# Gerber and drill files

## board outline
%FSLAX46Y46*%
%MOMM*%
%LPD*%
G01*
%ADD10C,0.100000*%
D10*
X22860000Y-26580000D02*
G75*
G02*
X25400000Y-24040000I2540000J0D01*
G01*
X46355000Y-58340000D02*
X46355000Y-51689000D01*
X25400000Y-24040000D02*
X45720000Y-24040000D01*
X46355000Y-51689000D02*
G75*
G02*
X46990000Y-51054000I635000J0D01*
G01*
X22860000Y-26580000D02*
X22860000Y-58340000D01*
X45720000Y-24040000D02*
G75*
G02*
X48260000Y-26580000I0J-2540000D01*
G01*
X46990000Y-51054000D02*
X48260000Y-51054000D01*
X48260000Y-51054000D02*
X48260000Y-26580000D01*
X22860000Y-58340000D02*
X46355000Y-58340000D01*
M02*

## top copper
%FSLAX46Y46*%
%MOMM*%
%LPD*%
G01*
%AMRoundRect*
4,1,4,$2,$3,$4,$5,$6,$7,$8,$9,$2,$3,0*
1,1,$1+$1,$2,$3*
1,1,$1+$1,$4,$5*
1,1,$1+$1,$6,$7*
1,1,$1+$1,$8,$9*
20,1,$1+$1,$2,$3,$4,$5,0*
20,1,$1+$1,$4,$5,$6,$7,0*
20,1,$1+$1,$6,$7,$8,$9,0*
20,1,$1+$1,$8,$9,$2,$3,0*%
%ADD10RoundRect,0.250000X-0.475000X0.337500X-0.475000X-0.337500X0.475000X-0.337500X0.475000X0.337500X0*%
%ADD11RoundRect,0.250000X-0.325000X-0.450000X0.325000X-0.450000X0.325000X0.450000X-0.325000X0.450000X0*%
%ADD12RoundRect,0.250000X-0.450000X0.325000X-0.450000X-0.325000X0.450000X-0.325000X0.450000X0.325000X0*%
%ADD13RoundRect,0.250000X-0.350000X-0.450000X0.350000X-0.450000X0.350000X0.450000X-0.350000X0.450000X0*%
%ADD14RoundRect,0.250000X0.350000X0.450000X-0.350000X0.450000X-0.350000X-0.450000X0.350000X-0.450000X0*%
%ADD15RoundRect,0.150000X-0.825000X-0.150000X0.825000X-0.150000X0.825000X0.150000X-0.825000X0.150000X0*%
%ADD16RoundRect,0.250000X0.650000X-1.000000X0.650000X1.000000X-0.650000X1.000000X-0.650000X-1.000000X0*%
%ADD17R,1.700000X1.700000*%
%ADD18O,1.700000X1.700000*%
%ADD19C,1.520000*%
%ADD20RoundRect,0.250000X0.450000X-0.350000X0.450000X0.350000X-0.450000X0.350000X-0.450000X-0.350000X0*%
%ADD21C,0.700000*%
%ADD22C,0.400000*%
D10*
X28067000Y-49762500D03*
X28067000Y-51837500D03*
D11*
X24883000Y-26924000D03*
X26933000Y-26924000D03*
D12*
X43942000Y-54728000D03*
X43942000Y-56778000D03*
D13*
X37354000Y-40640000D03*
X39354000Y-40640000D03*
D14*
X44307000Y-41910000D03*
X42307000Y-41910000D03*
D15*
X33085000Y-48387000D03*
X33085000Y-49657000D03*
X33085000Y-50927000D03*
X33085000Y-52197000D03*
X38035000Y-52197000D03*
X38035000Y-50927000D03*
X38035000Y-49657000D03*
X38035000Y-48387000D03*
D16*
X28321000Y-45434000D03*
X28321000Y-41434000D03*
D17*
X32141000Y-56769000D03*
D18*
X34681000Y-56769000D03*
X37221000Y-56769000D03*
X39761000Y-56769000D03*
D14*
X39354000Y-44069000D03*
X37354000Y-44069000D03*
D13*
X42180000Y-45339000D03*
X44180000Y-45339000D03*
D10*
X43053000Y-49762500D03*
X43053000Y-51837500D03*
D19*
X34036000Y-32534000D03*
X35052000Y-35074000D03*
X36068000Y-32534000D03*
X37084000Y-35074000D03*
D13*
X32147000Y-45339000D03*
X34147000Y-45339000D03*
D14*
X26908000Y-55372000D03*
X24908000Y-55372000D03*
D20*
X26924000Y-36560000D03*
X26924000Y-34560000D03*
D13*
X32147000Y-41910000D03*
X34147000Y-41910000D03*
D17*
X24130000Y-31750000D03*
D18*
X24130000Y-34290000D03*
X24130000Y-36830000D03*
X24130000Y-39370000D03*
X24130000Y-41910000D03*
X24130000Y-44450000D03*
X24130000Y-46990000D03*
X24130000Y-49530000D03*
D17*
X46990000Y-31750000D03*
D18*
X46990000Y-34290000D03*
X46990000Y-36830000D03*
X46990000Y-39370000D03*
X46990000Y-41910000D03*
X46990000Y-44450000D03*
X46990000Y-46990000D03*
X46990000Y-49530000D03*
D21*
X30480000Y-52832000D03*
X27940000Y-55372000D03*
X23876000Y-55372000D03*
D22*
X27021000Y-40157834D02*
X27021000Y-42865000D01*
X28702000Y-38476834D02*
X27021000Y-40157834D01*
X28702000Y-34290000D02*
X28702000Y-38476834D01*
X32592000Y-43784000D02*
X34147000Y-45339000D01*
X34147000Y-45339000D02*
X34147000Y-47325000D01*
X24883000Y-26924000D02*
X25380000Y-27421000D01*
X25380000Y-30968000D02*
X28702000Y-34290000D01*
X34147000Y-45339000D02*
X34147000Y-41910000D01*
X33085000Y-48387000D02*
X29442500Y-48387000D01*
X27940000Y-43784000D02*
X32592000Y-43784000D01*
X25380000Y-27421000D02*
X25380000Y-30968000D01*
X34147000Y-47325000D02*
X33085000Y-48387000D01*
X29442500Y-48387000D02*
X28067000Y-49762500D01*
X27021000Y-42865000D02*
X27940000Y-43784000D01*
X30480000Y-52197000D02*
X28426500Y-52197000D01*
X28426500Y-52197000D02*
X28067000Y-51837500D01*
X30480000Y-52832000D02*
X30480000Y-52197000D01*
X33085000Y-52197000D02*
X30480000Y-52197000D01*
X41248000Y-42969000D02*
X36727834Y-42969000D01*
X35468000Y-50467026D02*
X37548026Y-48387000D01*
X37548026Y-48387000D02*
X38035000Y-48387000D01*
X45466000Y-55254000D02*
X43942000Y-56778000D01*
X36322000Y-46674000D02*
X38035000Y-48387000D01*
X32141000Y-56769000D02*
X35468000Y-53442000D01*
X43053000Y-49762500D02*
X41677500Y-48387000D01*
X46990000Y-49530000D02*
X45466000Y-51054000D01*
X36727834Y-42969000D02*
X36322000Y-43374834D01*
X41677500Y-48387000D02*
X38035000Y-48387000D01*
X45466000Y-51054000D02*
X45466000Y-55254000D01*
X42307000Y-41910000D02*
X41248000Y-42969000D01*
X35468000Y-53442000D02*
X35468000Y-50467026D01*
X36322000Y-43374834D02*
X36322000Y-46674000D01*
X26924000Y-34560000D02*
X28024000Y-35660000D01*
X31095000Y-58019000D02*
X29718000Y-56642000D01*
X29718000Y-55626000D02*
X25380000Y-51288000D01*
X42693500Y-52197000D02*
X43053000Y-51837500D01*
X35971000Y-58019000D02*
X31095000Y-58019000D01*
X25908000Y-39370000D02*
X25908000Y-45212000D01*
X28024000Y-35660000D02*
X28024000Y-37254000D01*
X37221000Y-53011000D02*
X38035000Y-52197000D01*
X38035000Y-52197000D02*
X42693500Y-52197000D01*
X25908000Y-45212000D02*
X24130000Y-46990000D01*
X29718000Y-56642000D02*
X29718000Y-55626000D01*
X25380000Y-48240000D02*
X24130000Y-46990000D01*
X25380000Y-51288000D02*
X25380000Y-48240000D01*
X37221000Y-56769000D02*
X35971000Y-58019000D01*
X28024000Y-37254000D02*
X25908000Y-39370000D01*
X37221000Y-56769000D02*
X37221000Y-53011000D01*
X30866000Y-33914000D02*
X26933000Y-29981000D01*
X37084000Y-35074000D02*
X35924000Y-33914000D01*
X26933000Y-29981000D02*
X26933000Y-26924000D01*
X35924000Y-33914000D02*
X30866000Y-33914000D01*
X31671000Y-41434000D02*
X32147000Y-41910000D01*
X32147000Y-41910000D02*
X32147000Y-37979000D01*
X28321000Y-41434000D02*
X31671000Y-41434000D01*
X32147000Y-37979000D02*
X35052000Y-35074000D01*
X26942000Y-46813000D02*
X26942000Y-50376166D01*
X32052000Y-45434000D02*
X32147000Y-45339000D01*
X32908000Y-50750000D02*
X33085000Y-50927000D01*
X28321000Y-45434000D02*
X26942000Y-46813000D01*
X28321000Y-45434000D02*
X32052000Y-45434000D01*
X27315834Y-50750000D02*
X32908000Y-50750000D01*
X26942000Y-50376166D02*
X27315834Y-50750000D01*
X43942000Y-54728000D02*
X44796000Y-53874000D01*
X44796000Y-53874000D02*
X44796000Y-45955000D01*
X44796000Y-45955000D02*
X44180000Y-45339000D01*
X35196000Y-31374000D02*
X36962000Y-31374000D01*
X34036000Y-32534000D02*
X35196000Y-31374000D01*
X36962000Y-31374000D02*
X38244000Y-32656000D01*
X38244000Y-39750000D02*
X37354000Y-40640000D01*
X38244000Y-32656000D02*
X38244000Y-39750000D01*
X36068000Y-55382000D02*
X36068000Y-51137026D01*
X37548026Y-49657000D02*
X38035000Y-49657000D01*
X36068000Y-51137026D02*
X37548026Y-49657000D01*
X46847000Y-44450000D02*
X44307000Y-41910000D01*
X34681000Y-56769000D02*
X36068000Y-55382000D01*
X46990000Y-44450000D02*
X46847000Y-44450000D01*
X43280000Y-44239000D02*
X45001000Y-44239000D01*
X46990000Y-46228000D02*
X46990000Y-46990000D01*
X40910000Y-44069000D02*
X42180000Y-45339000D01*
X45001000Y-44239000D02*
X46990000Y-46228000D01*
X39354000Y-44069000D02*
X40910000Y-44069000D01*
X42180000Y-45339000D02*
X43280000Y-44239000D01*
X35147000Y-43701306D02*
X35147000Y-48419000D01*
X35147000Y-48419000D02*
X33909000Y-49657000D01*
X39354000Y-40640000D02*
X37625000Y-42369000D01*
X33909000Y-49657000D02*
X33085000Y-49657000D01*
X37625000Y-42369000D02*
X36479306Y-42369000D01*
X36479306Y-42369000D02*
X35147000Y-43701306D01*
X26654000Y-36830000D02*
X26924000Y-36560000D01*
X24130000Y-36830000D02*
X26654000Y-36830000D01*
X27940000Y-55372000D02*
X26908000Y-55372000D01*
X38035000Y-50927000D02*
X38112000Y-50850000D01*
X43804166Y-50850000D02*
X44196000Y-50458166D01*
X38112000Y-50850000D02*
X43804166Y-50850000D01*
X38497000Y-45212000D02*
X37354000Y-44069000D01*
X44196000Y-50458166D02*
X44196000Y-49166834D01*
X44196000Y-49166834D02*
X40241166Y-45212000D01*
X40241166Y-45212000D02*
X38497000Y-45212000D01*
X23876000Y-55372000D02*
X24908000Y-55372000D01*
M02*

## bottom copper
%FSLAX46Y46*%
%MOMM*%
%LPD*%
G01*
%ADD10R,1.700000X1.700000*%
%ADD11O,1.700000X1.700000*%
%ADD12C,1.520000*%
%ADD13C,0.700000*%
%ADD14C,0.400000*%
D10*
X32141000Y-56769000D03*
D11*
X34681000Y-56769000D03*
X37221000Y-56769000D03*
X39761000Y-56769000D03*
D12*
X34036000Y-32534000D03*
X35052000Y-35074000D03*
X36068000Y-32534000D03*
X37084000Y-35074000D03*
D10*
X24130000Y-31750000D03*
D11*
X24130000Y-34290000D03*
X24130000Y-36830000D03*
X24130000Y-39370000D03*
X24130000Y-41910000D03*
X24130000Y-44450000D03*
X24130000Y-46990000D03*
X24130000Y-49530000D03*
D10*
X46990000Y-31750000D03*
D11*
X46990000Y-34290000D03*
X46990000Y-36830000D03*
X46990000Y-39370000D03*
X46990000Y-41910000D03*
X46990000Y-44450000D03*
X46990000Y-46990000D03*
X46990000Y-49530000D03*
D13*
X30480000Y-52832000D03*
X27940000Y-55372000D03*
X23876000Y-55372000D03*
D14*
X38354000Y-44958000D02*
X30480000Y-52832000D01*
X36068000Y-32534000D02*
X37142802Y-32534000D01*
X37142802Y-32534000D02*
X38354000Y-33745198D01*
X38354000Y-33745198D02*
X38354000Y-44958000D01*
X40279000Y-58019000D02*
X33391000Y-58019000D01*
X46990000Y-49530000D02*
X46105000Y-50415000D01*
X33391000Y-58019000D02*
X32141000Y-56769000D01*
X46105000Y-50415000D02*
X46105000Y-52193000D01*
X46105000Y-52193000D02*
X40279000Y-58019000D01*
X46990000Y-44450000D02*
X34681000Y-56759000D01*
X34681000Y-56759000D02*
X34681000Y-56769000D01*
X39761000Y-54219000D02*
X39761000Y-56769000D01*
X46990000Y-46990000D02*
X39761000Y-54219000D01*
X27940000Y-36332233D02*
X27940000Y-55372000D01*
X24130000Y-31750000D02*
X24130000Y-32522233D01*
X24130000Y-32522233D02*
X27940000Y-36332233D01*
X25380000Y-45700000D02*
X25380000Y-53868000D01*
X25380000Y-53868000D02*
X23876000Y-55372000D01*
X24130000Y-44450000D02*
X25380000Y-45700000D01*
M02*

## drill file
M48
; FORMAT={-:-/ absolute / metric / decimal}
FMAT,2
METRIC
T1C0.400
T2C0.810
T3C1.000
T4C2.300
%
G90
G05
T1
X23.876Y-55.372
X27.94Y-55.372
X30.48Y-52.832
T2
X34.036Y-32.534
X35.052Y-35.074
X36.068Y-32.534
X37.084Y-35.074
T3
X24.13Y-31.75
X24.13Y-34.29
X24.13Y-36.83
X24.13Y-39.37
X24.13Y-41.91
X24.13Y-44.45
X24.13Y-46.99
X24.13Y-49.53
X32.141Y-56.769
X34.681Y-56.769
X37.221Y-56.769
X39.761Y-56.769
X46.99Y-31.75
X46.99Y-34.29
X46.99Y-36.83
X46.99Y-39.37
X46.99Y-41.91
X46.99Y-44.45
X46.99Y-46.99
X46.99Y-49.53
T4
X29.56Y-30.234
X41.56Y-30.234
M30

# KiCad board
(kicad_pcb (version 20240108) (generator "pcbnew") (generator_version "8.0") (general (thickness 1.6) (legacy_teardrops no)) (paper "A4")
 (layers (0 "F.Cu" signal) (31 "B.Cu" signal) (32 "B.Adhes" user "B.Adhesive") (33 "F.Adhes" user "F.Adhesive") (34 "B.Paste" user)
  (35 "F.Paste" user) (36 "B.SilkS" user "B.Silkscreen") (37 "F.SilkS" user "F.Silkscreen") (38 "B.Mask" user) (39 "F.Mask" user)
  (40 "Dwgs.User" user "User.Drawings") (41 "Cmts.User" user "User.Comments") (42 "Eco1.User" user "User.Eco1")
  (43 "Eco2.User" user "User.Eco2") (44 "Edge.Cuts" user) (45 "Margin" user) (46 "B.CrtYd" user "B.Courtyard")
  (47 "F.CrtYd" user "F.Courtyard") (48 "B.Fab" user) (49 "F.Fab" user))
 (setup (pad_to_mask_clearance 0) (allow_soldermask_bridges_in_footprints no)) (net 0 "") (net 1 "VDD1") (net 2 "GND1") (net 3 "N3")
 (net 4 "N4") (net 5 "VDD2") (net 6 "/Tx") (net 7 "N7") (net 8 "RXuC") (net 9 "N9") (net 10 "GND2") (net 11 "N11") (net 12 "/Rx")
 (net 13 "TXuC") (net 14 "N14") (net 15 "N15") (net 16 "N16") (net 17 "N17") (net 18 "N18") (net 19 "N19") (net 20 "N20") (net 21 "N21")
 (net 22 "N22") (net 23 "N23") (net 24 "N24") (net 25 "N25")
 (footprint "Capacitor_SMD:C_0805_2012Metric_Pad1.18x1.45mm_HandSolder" (layer "F.Cu") (at 28.067 50.8 -90)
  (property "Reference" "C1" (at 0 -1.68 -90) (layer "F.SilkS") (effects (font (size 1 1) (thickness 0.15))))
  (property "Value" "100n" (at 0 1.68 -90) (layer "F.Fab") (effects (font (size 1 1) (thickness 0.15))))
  (pad "1" smd roundrect (at -1.0375 0 270) (size 1.175 1.45) (layers "F.Cu" "F.Paste" "F.Mask") (roundrect_rratio 0.212766) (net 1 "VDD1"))
  (pad "2" smd roundrect (at 1.0375 0 270) (size 1.175 1.45) (layers "F.Cu" "F.Paste" "F.Mask") (roundrect_rratio 0.212766) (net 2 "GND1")))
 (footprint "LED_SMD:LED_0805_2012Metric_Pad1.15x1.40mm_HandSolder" (layer "F.Cu") (at 25.908 26.924)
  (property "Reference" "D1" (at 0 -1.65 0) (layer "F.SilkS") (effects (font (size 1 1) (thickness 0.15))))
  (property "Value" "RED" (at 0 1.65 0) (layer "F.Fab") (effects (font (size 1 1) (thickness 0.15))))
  (pad "1" smd roundrect (at -1.025 0) (size 1.15 1.4) (layers "F.Cu" "F.Paste" "F.Mask") (roundrect_rratio 0.217391) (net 1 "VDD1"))
  (pad "2" smd roundrect (at 1.025 0) (size 1.15 1.4) (layers "F.Cu" "F.Paste" "F.Mask") (roundrect_rratio 0.217391) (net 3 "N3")))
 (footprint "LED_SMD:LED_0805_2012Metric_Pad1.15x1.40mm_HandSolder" (layer "F.Cu") (at 43.942 55.753 -90)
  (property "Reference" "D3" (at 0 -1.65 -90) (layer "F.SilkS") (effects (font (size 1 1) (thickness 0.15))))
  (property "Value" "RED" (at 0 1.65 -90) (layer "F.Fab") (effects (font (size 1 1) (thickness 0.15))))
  (pad "1" smd roundrect (at -1.025 0 270) (size 1.15 1.4) (layers "F.Cu" "F.Paste" "F.Mask") (roundrect_rratio 0.217391) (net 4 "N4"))
  (pad "2" smd roundrect (at 1.025 0 270) (size 1.15 1.4) (layers "F.Cu" "F.Paste" "F.Mask") (roundrect_rratio 0.217391) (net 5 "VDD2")))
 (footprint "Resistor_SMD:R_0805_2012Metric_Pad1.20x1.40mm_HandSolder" (layer "F.Cu") (at 38.354 40.64)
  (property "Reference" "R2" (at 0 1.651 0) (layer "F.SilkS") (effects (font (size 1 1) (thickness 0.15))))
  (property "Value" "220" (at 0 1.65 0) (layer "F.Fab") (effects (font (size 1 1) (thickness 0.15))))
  (pad "1" smd roundrect (at -1 0) (size 1.2 1.4) (layers "F.Cu" "F.Paste" "F.Mask") (roundrect_rratio 0.208333) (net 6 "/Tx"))
  (pad "2" smd roundrect (at 1 0) (size 1.2 1.4) (layers "F.Cu" "F.Paste" "F.Mask") (roundrect_rratio 0.208333) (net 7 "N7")))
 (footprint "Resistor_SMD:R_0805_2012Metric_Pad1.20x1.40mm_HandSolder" (layer "F.Cu") (at 43.307 41.91 180)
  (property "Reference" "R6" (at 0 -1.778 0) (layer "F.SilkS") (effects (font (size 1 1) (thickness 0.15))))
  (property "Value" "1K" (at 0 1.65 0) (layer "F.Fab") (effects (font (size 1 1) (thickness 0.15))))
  (pad "1" smd roundrect (at -1 0 180) (size 1.2 1.4) (layers "F.Cu" "F.Paste" "F.Mask") (roundrect_rratio 0.208333) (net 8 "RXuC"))
  (pad "2" smd roundrect (at 1 0 180) (size 1.2 1.4) (layers "F.Cu" "F.Paste" "F.Mask") (roundrect_rratio 0.208333) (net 5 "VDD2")))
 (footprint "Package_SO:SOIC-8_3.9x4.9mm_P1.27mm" (layer "F.Cu") (at 35.56 50.292)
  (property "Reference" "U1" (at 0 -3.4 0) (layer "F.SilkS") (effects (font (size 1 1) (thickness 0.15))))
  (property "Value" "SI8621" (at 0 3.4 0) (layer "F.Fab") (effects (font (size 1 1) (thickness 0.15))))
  (pad "1" smd roundrect (at -2.475 -1.905) (size 1.95 0.6) (layers "F.Cu" "F.Paste" "F.Mask") (roundrect_rratio 0.25) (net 1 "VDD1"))
  (pad "2" smd roundrect (at -2.475 -0.635) (size 1.95 0.6) (layers "F.Cu" "F.Paste" "F.Mask") (roundrect_rratio 0.25) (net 7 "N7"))
  (pad "3" smd roundrect (at -2.475 0.635) (size 1.95 0.6) (layers "F.Cu" "F.Paste" "F.Mask") (roundrect_rratio 0.25) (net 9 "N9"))
  (pad "4" smd roundrect (at -2.475 1.905) (size 1.95 0.6) (layers "F.Cu" "F.Paste" "F.Mask") (roundrect_rratio 0.25) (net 2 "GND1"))
  (pad "5" smd roundrect (at 2.475 1.905) (size 1.95 0.6) (layers "F.Cu" "F.Paste" "F.Mask") (roundrect_rratio 0.25) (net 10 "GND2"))
  (pad "6" smd roundrect (at 2.475 0.635) (size 1.95 0.6) (layers "F.Cu" "F.Paste" "F.Mask") (roundrect_rratio 0.25) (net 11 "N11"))
  (pad "7" smd roundrect (at 2.475 -0.635) (size 1.95 0.6) (layers "F.Cu" "F.Paste" "F.Mask") (roundrect_rratio 0.25) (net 8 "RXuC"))
  (pad "8" smd roundrect (at 2.475 -1.905) (size 1.95 0.6) (layers "F.Cu" "F.Paste" "F.Mask") (roundrect_rratio 0.25) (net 5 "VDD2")))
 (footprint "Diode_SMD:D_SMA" (layer "F.Cu") (at 28.321 43.434 90)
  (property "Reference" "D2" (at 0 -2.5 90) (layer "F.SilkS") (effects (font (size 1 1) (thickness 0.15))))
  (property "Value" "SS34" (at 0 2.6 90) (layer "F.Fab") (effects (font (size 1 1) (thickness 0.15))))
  (pad "1" smd roundrect (at -2 0 90) (size 2.5 1.8) (layers "F.Cu" "F.Paste" "F.Mask") (roundrect_rratio 0.1388888889) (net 9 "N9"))
  (pad "2" smd roundrect (at 2 0 90) (size 2.5 1.8) (layers "F.Cu" "F.Paste" "F.Mask") (roundrect_rratio 0.1388888889) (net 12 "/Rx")))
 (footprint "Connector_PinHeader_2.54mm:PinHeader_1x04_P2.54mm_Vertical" (layer "F.Cu") (at 32.141 56.769 90)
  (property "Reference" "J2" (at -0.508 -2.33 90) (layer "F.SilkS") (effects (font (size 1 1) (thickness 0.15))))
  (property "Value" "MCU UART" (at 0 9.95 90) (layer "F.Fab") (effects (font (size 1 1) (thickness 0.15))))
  (pad "1" thru_hole rect (at 0 0 90) (size 1.7 1.7) (drill 1) (layers "*.Cu" "*.Mask") (remove_unused_layers no) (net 5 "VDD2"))
  (pad "2" thru_hole oval (at 0 2.54 90) (size 1.7 1.7) (drill 1) (layers "*.Cu" "*.Mask") (remove_unused_layers no) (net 8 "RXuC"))
  (pad "3" thru_hole oval (at 0 5.08 90) (size 1.7 1.7) (drill 1) (layers "*.Cu" "*.Mask") (remove_unused_layers no) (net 10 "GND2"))
  (pad "4" thru_hole oval (at 0 7.62 90) (size 1.7 1.7) (drill 1) (layers "*.Cu" "*.Mask") (remove_unused_layers no) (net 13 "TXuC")))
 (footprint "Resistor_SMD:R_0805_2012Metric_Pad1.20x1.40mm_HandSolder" (layer "F.Cu") (at 38.354 44.069 180)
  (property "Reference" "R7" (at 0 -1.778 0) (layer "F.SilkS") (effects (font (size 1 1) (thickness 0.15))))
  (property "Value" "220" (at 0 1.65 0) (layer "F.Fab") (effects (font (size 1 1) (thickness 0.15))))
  (pad "1" smd roundrect (at -1 0 180) (size 1.2 1.4) (layers "F.Cu" "F.Paste" "F.Mask") (roundrect_rratio 0.208333) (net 13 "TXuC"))
  (pad "2" smd roundrect (at 1 0 180) (size 1.2 1.4) (layers "F.Cu" "F.Paste" "F.Mask") (roundrect_rratio 0.208333) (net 11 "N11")))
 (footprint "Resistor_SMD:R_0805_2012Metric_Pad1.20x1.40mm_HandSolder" (layer "F.Cu") (at 43.18 45.339)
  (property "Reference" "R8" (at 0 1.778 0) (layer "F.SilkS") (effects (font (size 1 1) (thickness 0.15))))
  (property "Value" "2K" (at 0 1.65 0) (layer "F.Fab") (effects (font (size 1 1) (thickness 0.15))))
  (pad "1" smd roundrect (at -1 0) (size 1.2 1.4) (layers "F.Cu" "F.Paste" "F.Mask") (roundrect_rratio 0.208333) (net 13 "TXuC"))
  (pad "2" smd roundrect (at 1 0) (size 1.2 1.4) (layers "F.Cu" "F.Paste" "F.Mask") (roundrect_rratio 0.208333) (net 4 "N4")))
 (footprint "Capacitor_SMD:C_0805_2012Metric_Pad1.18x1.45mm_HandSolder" (layer "F.Cu") (at 43.053 50.8 -90)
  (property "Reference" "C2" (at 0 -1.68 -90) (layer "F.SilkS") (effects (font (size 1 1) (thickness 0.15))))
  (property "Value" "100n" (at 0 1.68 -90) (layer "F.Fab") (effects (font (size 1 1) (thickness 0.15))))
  (pad "1" smd roundrect (at -1.0375 0 270) (size 1.175 1.45) (layers "F.Cu" "F.Paste" "F.Mask") (roundrect_rratio 0.212766) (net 5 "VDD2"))
  (pad "2" smd roundrect (at 1.0375 0 270) (size 1.175 1.45) (layers "F.Cu" "F.Paste" "F.Mask") (roundrect_rratio 0.212766) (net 10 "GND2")))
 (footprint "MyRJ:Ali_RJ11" (layer "F.Cu") (at 34.036 32.534 180)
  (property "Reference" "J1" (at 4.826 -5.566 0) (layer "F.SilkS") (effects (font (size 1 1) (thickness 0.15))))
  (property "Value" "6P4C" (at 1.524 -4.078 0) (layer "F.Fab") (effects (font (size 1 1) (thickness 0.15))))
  (pad "" np_thru_hole circle (at -7.524 2.3 180) (size 2.3 2.3) (drill 2.3) (layers "F&B.Cu" "*.Mask"))
  (pad "" np_thru_hole circle (at 4.476 2.3 180) (size 2.3 2.3) (drill 2.3) (layers "F&B.Cu" "*.Mask"))
  (pad "1" thru_hole circle (at 0 0) (size 1.52 1.52) (drill 0.81) (layers "*.Cu" "*.Mask") (remove_unused_layers no) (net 6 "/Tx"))
  (pad "2" thru_hole circle (at -1.016 -2.54) (size 1.52 1.52) (drill 0.81) (layers "*.Cu" "*.Mask") (remove_unused_layers no)
   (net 12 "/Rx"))
  (pad "3" thru_hole circle (at -2.032 0) (size 1.52 1.52) (drill 0.81) (layers "*.Cu" "*.Mask") (remove_unused_layers no) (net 2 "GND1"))
  (pad "4" thru_hole circle (at -3.048 -2.54) (size 1.52 1.52) (drill 0.81) (layers "*.Cu" "*.Mask") (remove_unused_layers no) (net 3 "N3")))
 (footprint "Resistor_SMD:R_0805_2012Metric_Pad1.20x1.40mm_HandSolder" (layer "F.Cu") (at 33.147 45.339)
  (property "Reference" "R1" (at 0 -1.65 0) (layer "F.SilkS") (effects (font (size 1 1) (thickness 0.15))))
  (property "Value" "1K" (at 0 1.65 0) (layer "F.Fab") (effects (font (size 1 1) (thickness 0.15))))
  (pad "1" smd roundrect (at -1 0) (size 1.2 1.4) (layers "F.Cu" "F.Paste" "F.Mask") (roundrect_rratio 0.208333) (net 9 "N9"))
  (pad "2" smd roundrect (at 1 0) (size 1.2 1.4) (layers "F.Cu" "F.Paste" "F.Mask") (roundrect_rratio 0.208333) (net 1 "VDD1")))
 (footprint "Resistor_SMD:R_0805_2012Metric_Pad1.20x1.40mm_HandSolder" (layer "F.Cu") (at 25.908 55.372 180)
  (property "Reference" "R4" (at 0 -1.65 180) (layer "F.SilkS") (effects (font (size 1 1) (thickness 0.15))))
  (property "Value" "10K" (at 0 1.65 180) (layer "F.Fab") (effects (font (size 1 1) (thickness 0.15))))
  (pad "1" smd roundrect (at -1 0 180) (size 1.2 1.4) (layers "F.Cu" "F.Paste" "F.Mask") (roundrect_rratio 0.208333) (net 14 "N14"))
  (pad "2" smd roundrect (at 1 0 180) (size 1.2 1.4) (layers "F.Cu" "F.Paste" "F.Mask") (roundrect_rratio 0.208333) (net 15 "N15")))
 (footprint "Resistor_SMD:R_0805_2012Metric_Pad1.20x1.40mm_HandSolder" (layer "F.Cu") (at 26.924 35.56 90)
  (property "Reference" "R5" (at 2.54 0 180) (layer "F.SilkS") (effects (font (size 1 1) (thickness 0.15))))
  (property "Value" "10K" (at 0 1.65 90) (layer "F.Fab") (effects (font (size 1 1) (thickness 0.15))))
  (pad "1" smd roundrect (at -1 0 90) (size 1.2 1.4) (layers "F.Cu" "F.Paste" "F.Mask") (roundrect_rratio 0.208333) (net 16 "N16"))
  (pad "2" smd roundrect (at 1 0 90) (size 1.2 1.4) (layers "F.Cu" "F.Paste" "F.Mask") (roundrect_rratio 0.208333) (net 10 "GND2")))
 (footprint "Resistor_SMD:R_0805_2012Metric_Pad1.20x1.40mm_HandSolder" (layer "F.Cu") (at 33.147 41.91)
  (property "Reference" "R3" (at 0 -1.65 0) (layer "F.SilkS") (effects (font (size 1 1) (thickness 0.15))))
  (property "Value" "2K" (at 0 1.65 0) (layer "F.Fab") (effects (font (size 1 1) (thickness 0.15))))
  (pad "1" smd roundrect (at -1 0) (size 1.2 1.4) (layers "F.Cu" "F.Paste" "F.Mask") (roundrect_rratio 0.208333) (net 12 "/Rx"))
  (pad "2" smd roundrect (at 1 0) (size 1.2 1.4) (layers "F.Cu" "F.Paste" "F.Mask") (roundrect_rratio 0.208333) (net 1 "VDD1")))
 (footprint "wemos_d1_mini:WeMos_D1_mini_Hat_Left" (layer "B.Cu") (at 24.13 31.75 180)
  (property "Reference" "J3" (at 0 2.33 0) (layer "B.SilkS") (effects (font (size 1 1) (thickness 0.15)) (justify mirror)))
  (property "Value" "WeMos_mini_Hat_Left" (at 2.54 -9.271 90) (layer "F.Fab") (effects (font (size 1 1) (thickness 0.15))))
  (pad "1" thru_hole rect (at 0 0 180) (size 1.7 1.7) (drill 1) (layers "*.Cu" "*.Mask") (remove_unused_layers no) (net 14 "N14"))
  (pad "2" thru_hole oval (at 0 -2.54 180) (size 1.7 1.7) (drill 1) (layers "*.Cu" "*.Mask") (remove_unused_layers no) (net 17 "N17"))
  (pad "3" thru_hole oval (at 0 -5.08 180) (size 1.7 1.7) (drill 1) (layers "*.Cu" "*.Mask") (remove_unused_layers no) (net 16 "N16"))
  (pad "4" thru_hole oval (at 0 -7.62 180) (size 1.7 1.7) (drill 1) (layers "*.Cu" "*.Mask") (remove_unused_layers no) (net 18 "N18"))
  (pad "5" thru_hole oval (at 0 -10.16 180) (size 1.7 1.7) (drill 1) (layers "*.Cu" "*.Mask") (remove_unused_layers no) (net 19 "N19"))
  (pad "6" thru_hole oval (at 0 -12.7 180) (size 1.7 1.7) (drill 1) (layers "*.Cu" "*.Mask") (remove_unused_layers no) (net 15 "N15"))
  (pad "7" thru_hole oval (at 0 -15.24 180) (size 1.7 1.7) (drill 1) (layers "*.Cu" "*.Mask") (remove_unused_layers no) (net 10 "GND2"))
  (pad "8" thru_hole oval (at 0 -17.78 180) (size 1.7 1.7) (drill 1) (layers "*.Cu" "*.Mask") (remove_unused_layers no) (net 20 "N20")))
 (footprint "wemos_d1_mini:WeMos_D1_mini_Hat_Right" (layer "B.Cu") (at 46.99 31.75 180)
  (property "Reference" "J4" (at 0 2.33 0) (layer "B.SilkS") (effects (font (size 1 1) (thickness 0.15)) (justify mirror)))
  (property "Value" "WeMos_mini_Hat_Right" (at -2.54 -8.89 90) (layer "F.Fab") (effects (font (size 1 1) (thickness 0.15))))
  (pad "1" thru_hole rect (at 0 0 180) (size 1.7 1.7) (drill 1) (layers "*.Cu" "*.Mask") (remove_unused_layers no) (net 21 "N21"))
  (pad "2" thru_hole oval (at 0 -2.54 180) (size 1.7 1.7) (drill 1) (layers "*.Cu" "*.Mask") (remove_unused_layers no) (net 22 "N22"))
  (pad "3" thru_hole oval (at 0 -5.08 180) (size 1.7 1.7) (drill 1) (layers "*.Cu" "*.Mask") (remove_unused_layers no) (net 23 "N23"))
  (pad "4" thru_hole oval (at 0 -7.62 180) (size 1.7 1.7) (drill 1) (layers "*.Cu" "*.Mask") (remove_unused_layers no) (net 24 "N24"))
  (pad "5" thru_hole oval (at 0 -10.16 180) (size 1.7 1.7) (drill 1) (layers "*.Cu" "*.Mask") (remove_unused_layers no) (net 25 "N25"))
  (pad "6" thru_hole oval (at 0 -12.7 180) (size 1.7 1.7) (drill 1) (layers "*.Cu" "*.Mask") (remove_unused_layers no) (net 8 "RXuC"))
  (pad "7" thru_hole oval (at 0 -15.24 180) (size 1.7 1.7) (drill 1) (layers "*.Cu" "*.Mask") (remove_unused_layers no) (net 13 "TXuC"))
  (pad "8" thru_hole oval (at 0 -17.78 180) (size 1.7 1.7) (drill 1) (layers "*.Cu" "*.Mask") (remove_unused_layers no) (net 5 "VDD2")))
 (gr_arc (start 22.86 26.58) (mid 23.603949 24.783949) (end 25.4 24.04) (stroke (width 0.1) (type default)) (layer "Edge.Cuts"))
 (gr_line (start 46.355 58.34) (end 46.355 51.689) (stroke (width 0.1) (type default)) (layer "Edge.Cuts"))
 (gr_line (start 25.4 24.04) (end 45.72 24.04) (stroke (width 0.1) (type default)) (layer "Edge.Cuts"))
 (gr_arc (start 46.355 51.689) (mid 46.540987 51.239987) (end 46.99 51.054) (stroke (width 0.1) (type default)) (layer "Edge.Cuts"))
 (gr_line (start 22.86 26.58) (end 22.86 58.34) (stroke (width 0.1) (type default)) (layer "Edge.Cuts"))
 (gr_arc (start 45.72 24.04) (mid 47.516051 24.783949) (end 48.26 26.58) (stroke (width 0.1) (type default)) (layer "Edge.Cuts"))
 (gr_line (start 46.99 51.054) (end 48.26 51.054) (stroke (width 0.1) (type default)) (layer "Edge.Cuts"))
 (gr_line (start 48.26 51.054) (end 48.26 26.58) (stroke (width 0.1) (type default)) (layer "Edge.Cuts"))
 (gr_line (start 22.86 58.34) (end 46.355 58.34) (stroke (width 0.1) (type default)) (layer "Edge.Cuts"))
 (segment (start 27.021 40.157834) (end 27.021 42.865) (width 0.4) (layer "F.Cu") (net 1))
 (segment (start 28.702 38.476834) (end 27.021 40.157834) (width 0.4) (layer "F.Cu") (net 1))
 (segment (start 28.702 34.29) (end 28.702 38.476834) (width 0.4) (layer "F.Cu") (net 1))
 (segment (start 32.592 43.784) (end 34.147 45.339) (width 0.4) (layer "F.Cu") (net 1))
 (segment (start 34.147 45.339) (end 34.147 47.325) (width 0.4) (layer "F.Cu") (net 1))
 (segment (start 24.883 26.924) (end 25.38 27.421) (width 0.4) (layer "F.Cu") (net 1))
 (segment (start 25.38 30.968) (end 28.702 34.29) (width 0.4) (layer "F.Cu") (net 1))
 (segment (start 34.147 45.339) (end 34.147 41.91) (width 0.4) (layer "F.Cu") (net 1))
 (segment (start 33.085 48.387) (end 29.4425 48.387) (width 0.4) (layer "F.Cu") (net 1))
 (segment (start 27.94 43.784) (end 32.592 43.784) (width 0.4) (layer "F.Cu") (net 1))
 (segment (start 25.38 27.421) (end 25.38 30.968) (width 0.4) (layer "F.Cu") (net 1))
 (segment (start 34.147 47.325) (end 33.085 48.387) (width 0.4) (layer "F.Cu") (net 1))
 (segment (start 29.4425 48.387) (end 28.067 49.7625) (width 0.4) (layer "F.Cu") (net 1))
 (segment (start 27.021 42.865) (end 27.94 43.784) (width 0.4) (layer "F.Cu") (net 1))
 (segment (start 30.48 52.197) (end 28.4265 52.197) (width 0.4) (layer "F.Cu") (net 2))
 (segment (start 28.4265 52.197) (end 28.067 51.8375) (width 0.4) (layer "F.Cu") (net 2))
 (segment (start 30.48 52.832) (end 30.48 52.197) (width 0.4) (layer "F.Cu") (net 2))
 (segment (start 33.085 52.197) (end 30.48 52.197) (width 0.4) (layer "F.Cu") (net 2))
 (via (at 30.48 52.832) (size 0.7) (drill 0.4) (layers "F.Cu" "B.Cu") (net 2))
 (segment (start 38.354 44.958) (end 30.48 52.832) (width 0.4) (layer "B.Cu") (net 2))
 (segment (start 36.068 32.534) (end 37.142802 32.534) (width 0.4) (layer "B.Cu") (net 2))
 (segment (start 37.142802 32.534) (end 38.354 33.745198) (width 0.4) (layer "B.Cu") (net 2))
 (segment (start 38.354 33.745198) (end 38.354 44.958) (width 0.4) (layer "B.Cu") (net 2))
 (segment (start 41.248 42.969) (end 36.727834 42.969) (width 0.4) (layer "F.Cu") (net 5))
 (segment (start 35.468 50.467026) (end 37.548026 48.387) (width 0.4) (layer "F.Cu") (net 5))
 (segment (start 37.548026 48.387) (end 38.035 48.387) (width 0.4) (layer "F.Cu") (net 5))
 (segment (start 45.466 55.254) (end 43.942 56.778) (width 0.4) (layer "F.Cu") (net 5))
 (segment (start 36.322 46.674) (end 38.035 48.387) (width 0.4) (layer "F.Cu") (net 5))
 (segment (start 32.141 56.769) (end 35.468 53.442) (width 0.4) (layer "F.Cu") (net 5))
 (segment (start 43.053 49.7625) (end 41.6775 48.387) (width 0.4) (layer "F.Cu") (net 5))
 (segment (start 46.99 49.53) (end 45.466 51.054) (width 0.4) (layer "F.Cu") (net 5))
 (segment (start 36.727834 42.969) (end 36.322 43.374834) (width 0.4) (layer "F.Cu") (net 5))
 (segment (start 41.6775 48.387) (end 38.035 48.387) (width 0.4) (layer "F.Cu") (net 5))
 (segment (start 45.466 51.054) (end 45.466 55.254) (width 0.4) (layer "F.Cu") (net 5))
 (segment (start 42.307 41.91) (end 41.248 42.969) (width 0.4) (layer "F.Cu") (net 5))
 (segment (start 35.468 53.442) (end 35.468 50.467026) (width 0.4) (layer "F.Cu") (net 5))
 (segment (start 36.322 43.374834) (end 36.322 46.674) (width 0.4) (layer "F.Cu") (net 5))
 (segment (start 40.279 58.019) (end 33.391 58.019) (width 0.4) (layer "B.Cu") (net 5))
 (segment (start 46.99 49.53) (end 46.105 50.415) (width 0.4) (layer "B.Cu") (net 5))
 (segment (start 33.391 58.019) (end 32.141 56.769) (width 0.4) (layer "B.Cu") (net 5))
 (segment (start 46.105 50.415) (end 46.105 52.193) (width 0.4) (layer "B.Cu") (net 5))
 (segment (start 46.105 52.193) (end 40.279 58.019) (width 0.4) (layer "B.Cu") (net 5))
 (segment (start 26.924 34.56) (end 28.024 35.66) (width 0.4) (layer "F.Cu") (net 10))
 (segment (start 31.095 58.019) (end 29.718 56.642) (width 0.4) (layer "F.Cu") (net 10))
 (segment (start 29.718 55.626) (end 25.38 51.288) (width 0.4) (layer "F.Cu") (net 10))
 (segment (start 42.6935 52.197) (end 43.053 51.8375) (width 0.4) (layer "F.Cu") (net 10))
 (segment (start 35.971 58.019) (end 31.095 58.019) (width 0.4) (layer "F.Cu") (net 10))
 (segment (start 25.908 39.37) (end 25.908 45.212) (width 0.4) (layer "F.Cu") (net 10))
 (segment (start 28.024 35.66) (end 28.024 37.254) (width 0.4) (layer "F.Cu") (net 10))
 (segment (start 37.221 53.011) (end 38.035 52.197) (width 0.4) (layer "F.Cu") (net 10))
 (segment (start 38.035 52.197) (end 42.6935 52.197) (width 0.4) (layer "F.Cu") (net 10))
 (segment (start 25.908 45.212) (end 24.13 46.99) (width 0.4) (layer "F.Cu") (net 10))
 (segment (start 29.718 56.642) (end 29.718 55.626) (width 0.4) (layer "F.Cu") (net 10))
 (segment (start 25.38 48.24) (end 24.13 46.99) (width 0.4) (layer "F.Cu") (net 10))
 (segment (start 25.38 51.288) (end 25.38 48.24) (width 0.4) (layer "F.Cu") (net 10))
 (segment (start 37.221 56.769) (end 35.971 58.019) (width 0.4) (layer "F.Cu") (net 10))
 (segment (start 28.024 37.254) (end 25.908 39.37) (width 0.4) (layer "F.Cu") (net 10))
 (segment (start 37.221 56.769) (end 37.221 53.011) (width 0.4) (layer "F.Cu") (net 10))
 (segment (start 30.866 33.914) (end 26.933 29.981) (width 0.4) (layer "F.Cu") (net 3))
 (segment (start 37.084 35.074) (end 35.924 33.914) (width 0.4) (layer "F.Cu") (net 3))
 (segment (start 26.933 29.981) (end 26.933 26.924) (width 0.4) (layer "F.Cu") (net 3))
 (segment (start 35.924 33.914) (end 30.866 33.914) (width 0.4) (layer "F.Cu") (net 3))
 (segment (start 31.671 41.434) (end 32.147 41.91) (width 0.4) (layer "F.Cu") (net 12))
 (segment (start 32.147 41.91) (end 32.147 37.979) (width 0.4) (layer "F.Cu") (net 12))
 (segment (start 28.321 41.434) (end 31.671 41.434) (width 0.4) (layer "F.Cu") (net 12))
 (segment (start 32.147 37.979) (end 35.052 35.074) (width 0.4) (layer "F.Cu") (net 12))
 (segment (start 26.942 46.813) (end 26.942 50.376166) (width 0.4) (layer "F.Cu") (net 9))
 (segment (start 32.052 45.434) (end 32.147 45.339) (width 0.4) (layer "F.Cu") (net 9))
 (segment (start 32.908 50.75) (end 33.085 50.927) (width 0.4) (layer "F.Cu") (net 9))
 (segment (start 28.321 45.434) (end 26.942 46.813) (width 0.4) (layer "F.Cu") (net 9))
 (segment (start 28.321 45.434) (end 32.052 45.434) (width 0.4) (layer "F.Cu") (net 9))
 (segment (start 27.315834 50.75) (end 32.908 50.75) (width 0.4) (layer "F.Cu") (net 9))
 (segment (start 26.942 50.376166) (end 27.315834 50.75) (width 0.4) (layer "F.Cu") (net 9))
 (segment (start 43.942 54.728) (end 44.796 53.874) (width 0.4) (layer "F.Cu") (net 4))
 (segment (start 44.796 53.874) (end 44.796 45.955) (width 0.4) (layer "F.Cu") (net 4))
 (segment (start 44.796 45.955) (end 44.18 45.339) (width 0.4) (layer "F.Cu") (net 4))
 (segment (start 35.196 31.374) (end 36.962 31.374) (width 0.4) (layer "F.Cu") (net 6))
 (segment (start 34.036 32.534) (end 35.196 31.374) (width 0.4) (layer "F.Cu") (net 6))
 (segment (start 36.962 31.374) (end 38.244 32.656) (width 0.4) (layer "F.Cu") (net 6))
 (segment (start 38.244 39.75) (end 37.354 40.64) (width 0.4) (layer "F.Cu") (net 6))
 (segment (start 38.244 32.656) (end 38.244 39.75) (width 0.4) (layer "F.Cu") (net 6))
 (segment (start 36.068 55.382) (end 36.068 51.137026) (width 0.4) (layer "F.Cu") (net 8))
 (segment (start 37.548026 49.657) (end 38.035 49.657) (width 0.4) (layer "F.Cu") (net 8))
 (segment (start 36.068 51.137026) (end 37.548026 49.657) (width 0.4) (layer "F.Cu") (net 8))
 (segment (start 46.847 44.45) (end 44.307 41.91) (width 0.4) (layer "F.Cu") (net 8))
 (segment (start 34.681 56.769) (end 36.068 55.382) (width 0.4) (layer "F.Cu") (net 8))
 (segment (start 46.99 44.45) (end 46.847 44.45) (width 0.4) (layer "F.Cu") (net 8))
 (segment (start 46.99 44.45) (end 34.681 56.759) (width 0.4) (layer "B.Cu") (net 8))
 (segment (start 34.681 56.759) (end 34.681 56.769) (width 0.4) (layer "B.Cu") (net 8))
 (segment (start 43.28 44.239) (end 45.001 44.239) (width 0.4) (layer "F.Cu") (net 13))
 (segment (start 46.99 46.228) (end 46.99 46.99) (width 0.4) (layer "F.Cu") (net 13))
 (segment (start 40.91 44.069) (end 42.18 45.339) (width 0.4) (layer "F.Cu") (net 13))
 (segment (start 45.001 44.239) (end 46.99 46.228) (width 0.4) (layer "F.Cu") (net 13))
 (segment (start 39.354 44.069) (end 40.91 44.069) (width 0.4) (layer "F.Cu") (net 13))
 (segment (start 42.18 45.339) (end 43.28 44.239) (width 0.4) (layer "F.Cu") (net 13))
 (segment (start 39.761 54.219) (end 39.761 56.769) (width 0.4) (layer "B.Cu") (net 13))
 (segment (start 46.99 46.99) (end 39.761 54.219) (width 0.4) (layer "B.Cu") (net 13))
 (segment (start 35.147 43.701306) (end 35.147 48.419) (width 0.4) (layer "F.Cu") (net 7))
 (segment (start 35.147 48.419) (end 33.909 49.657) (width 0.4) (layer "F.Cu") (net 7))
 (segment (start 39.354 40.64) (end 37.625 42.369) (width 0.4) (layer "F.Cu") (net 7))
 (segment (start 33.909 49.657) (end 33.085 49.657) (width 0.4) (layer "F.Cu") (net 7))
 (segment (start 37.625 42.369) (end 36.479306 42.369) (width 0.4) (layer "F.Cu") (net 7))
 (segment (start 36.479306 42.369) (end 35.147 43.701306) (width 0.4) (layer "F.Cu") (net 7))
 (segment (start 26.654 36.83) (end 26.924 36.56) (width 0.4) (layer "F.Cu") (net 16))
 (segment (start 24.13 36.83) (end 26.654 36.83) (width 0.4) (layer "F.Cu") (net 16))
 (segment (start 27.94 55.372) (end 26.908 55.372) (width 0.4) (layer "F.Cu") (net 14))
 (via (at 27.94 55.372) (size 0.7) (drill 0.4) (layers "F.Cu" "B.Cu") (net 14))
 (segment (start 27.94 36.332233) (end 27.94 55.372) (width 0.4) (layer "B.Cu") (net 14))
 (segment (start 24.13 31.75) (end 24.13 32.522233) (width 0.4) (layer "B.Cu") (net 14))
 (segment (start 24.13 32.522233) (end 27.94 36.332233) (width 0.4) (layer "B.Cu") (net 14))
 (segment (start 38.035 50.927) (end 38.112 50.85) (width 0.4) (layer "F.Cu") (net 11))
 (segment (start 43.804166 50.85) (end 44.196 50.458166) (width 0.4) (layer "F.Cu") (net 11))
 (segment (start 38.112 50.85) (end 43.804166 50.85) (width 0.4) (layer "F.Cu") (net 11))
 (segment (start 38.497 45.212) (end 37.354 44.069) (width 0.4) (layer "F.Cu") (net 11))
 (segment (start 44.196 50.458166) (end 44.196 49.166834) (width 0.4) (layer "F.Cu") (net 11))
 (segment (start 44.196 49.166834) (end 40.241166 45.212) (width 0.4) (layer "F.Cu") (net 11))
 (segment (start 40.241166 45.212) (end 38.497 45.212) (width 0.4) (layer "F.Cu") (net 11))
 (segment (start 23.876 55.372) (end 24.908 55.372) (width 0.4) (layer "F.Cu") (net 15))
 (via (at 23.876 55.372) (size 0.7) (drill 0.4) (layers "F.Cu" "B.Cu") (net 15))
 (segment (start 25.38 45.7) (end 25.38 53.868) (width 0.4) (layer "B.Cu") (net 15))
 (segment (start 25.38 53.868) (end 23.876 55.372) (width 0.4) (layer "B.Cu") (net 15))
 (segment (start 24.13 44.45) (end 25.38 45.7) (width 0.4) (layer "B.Cu") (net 15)))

